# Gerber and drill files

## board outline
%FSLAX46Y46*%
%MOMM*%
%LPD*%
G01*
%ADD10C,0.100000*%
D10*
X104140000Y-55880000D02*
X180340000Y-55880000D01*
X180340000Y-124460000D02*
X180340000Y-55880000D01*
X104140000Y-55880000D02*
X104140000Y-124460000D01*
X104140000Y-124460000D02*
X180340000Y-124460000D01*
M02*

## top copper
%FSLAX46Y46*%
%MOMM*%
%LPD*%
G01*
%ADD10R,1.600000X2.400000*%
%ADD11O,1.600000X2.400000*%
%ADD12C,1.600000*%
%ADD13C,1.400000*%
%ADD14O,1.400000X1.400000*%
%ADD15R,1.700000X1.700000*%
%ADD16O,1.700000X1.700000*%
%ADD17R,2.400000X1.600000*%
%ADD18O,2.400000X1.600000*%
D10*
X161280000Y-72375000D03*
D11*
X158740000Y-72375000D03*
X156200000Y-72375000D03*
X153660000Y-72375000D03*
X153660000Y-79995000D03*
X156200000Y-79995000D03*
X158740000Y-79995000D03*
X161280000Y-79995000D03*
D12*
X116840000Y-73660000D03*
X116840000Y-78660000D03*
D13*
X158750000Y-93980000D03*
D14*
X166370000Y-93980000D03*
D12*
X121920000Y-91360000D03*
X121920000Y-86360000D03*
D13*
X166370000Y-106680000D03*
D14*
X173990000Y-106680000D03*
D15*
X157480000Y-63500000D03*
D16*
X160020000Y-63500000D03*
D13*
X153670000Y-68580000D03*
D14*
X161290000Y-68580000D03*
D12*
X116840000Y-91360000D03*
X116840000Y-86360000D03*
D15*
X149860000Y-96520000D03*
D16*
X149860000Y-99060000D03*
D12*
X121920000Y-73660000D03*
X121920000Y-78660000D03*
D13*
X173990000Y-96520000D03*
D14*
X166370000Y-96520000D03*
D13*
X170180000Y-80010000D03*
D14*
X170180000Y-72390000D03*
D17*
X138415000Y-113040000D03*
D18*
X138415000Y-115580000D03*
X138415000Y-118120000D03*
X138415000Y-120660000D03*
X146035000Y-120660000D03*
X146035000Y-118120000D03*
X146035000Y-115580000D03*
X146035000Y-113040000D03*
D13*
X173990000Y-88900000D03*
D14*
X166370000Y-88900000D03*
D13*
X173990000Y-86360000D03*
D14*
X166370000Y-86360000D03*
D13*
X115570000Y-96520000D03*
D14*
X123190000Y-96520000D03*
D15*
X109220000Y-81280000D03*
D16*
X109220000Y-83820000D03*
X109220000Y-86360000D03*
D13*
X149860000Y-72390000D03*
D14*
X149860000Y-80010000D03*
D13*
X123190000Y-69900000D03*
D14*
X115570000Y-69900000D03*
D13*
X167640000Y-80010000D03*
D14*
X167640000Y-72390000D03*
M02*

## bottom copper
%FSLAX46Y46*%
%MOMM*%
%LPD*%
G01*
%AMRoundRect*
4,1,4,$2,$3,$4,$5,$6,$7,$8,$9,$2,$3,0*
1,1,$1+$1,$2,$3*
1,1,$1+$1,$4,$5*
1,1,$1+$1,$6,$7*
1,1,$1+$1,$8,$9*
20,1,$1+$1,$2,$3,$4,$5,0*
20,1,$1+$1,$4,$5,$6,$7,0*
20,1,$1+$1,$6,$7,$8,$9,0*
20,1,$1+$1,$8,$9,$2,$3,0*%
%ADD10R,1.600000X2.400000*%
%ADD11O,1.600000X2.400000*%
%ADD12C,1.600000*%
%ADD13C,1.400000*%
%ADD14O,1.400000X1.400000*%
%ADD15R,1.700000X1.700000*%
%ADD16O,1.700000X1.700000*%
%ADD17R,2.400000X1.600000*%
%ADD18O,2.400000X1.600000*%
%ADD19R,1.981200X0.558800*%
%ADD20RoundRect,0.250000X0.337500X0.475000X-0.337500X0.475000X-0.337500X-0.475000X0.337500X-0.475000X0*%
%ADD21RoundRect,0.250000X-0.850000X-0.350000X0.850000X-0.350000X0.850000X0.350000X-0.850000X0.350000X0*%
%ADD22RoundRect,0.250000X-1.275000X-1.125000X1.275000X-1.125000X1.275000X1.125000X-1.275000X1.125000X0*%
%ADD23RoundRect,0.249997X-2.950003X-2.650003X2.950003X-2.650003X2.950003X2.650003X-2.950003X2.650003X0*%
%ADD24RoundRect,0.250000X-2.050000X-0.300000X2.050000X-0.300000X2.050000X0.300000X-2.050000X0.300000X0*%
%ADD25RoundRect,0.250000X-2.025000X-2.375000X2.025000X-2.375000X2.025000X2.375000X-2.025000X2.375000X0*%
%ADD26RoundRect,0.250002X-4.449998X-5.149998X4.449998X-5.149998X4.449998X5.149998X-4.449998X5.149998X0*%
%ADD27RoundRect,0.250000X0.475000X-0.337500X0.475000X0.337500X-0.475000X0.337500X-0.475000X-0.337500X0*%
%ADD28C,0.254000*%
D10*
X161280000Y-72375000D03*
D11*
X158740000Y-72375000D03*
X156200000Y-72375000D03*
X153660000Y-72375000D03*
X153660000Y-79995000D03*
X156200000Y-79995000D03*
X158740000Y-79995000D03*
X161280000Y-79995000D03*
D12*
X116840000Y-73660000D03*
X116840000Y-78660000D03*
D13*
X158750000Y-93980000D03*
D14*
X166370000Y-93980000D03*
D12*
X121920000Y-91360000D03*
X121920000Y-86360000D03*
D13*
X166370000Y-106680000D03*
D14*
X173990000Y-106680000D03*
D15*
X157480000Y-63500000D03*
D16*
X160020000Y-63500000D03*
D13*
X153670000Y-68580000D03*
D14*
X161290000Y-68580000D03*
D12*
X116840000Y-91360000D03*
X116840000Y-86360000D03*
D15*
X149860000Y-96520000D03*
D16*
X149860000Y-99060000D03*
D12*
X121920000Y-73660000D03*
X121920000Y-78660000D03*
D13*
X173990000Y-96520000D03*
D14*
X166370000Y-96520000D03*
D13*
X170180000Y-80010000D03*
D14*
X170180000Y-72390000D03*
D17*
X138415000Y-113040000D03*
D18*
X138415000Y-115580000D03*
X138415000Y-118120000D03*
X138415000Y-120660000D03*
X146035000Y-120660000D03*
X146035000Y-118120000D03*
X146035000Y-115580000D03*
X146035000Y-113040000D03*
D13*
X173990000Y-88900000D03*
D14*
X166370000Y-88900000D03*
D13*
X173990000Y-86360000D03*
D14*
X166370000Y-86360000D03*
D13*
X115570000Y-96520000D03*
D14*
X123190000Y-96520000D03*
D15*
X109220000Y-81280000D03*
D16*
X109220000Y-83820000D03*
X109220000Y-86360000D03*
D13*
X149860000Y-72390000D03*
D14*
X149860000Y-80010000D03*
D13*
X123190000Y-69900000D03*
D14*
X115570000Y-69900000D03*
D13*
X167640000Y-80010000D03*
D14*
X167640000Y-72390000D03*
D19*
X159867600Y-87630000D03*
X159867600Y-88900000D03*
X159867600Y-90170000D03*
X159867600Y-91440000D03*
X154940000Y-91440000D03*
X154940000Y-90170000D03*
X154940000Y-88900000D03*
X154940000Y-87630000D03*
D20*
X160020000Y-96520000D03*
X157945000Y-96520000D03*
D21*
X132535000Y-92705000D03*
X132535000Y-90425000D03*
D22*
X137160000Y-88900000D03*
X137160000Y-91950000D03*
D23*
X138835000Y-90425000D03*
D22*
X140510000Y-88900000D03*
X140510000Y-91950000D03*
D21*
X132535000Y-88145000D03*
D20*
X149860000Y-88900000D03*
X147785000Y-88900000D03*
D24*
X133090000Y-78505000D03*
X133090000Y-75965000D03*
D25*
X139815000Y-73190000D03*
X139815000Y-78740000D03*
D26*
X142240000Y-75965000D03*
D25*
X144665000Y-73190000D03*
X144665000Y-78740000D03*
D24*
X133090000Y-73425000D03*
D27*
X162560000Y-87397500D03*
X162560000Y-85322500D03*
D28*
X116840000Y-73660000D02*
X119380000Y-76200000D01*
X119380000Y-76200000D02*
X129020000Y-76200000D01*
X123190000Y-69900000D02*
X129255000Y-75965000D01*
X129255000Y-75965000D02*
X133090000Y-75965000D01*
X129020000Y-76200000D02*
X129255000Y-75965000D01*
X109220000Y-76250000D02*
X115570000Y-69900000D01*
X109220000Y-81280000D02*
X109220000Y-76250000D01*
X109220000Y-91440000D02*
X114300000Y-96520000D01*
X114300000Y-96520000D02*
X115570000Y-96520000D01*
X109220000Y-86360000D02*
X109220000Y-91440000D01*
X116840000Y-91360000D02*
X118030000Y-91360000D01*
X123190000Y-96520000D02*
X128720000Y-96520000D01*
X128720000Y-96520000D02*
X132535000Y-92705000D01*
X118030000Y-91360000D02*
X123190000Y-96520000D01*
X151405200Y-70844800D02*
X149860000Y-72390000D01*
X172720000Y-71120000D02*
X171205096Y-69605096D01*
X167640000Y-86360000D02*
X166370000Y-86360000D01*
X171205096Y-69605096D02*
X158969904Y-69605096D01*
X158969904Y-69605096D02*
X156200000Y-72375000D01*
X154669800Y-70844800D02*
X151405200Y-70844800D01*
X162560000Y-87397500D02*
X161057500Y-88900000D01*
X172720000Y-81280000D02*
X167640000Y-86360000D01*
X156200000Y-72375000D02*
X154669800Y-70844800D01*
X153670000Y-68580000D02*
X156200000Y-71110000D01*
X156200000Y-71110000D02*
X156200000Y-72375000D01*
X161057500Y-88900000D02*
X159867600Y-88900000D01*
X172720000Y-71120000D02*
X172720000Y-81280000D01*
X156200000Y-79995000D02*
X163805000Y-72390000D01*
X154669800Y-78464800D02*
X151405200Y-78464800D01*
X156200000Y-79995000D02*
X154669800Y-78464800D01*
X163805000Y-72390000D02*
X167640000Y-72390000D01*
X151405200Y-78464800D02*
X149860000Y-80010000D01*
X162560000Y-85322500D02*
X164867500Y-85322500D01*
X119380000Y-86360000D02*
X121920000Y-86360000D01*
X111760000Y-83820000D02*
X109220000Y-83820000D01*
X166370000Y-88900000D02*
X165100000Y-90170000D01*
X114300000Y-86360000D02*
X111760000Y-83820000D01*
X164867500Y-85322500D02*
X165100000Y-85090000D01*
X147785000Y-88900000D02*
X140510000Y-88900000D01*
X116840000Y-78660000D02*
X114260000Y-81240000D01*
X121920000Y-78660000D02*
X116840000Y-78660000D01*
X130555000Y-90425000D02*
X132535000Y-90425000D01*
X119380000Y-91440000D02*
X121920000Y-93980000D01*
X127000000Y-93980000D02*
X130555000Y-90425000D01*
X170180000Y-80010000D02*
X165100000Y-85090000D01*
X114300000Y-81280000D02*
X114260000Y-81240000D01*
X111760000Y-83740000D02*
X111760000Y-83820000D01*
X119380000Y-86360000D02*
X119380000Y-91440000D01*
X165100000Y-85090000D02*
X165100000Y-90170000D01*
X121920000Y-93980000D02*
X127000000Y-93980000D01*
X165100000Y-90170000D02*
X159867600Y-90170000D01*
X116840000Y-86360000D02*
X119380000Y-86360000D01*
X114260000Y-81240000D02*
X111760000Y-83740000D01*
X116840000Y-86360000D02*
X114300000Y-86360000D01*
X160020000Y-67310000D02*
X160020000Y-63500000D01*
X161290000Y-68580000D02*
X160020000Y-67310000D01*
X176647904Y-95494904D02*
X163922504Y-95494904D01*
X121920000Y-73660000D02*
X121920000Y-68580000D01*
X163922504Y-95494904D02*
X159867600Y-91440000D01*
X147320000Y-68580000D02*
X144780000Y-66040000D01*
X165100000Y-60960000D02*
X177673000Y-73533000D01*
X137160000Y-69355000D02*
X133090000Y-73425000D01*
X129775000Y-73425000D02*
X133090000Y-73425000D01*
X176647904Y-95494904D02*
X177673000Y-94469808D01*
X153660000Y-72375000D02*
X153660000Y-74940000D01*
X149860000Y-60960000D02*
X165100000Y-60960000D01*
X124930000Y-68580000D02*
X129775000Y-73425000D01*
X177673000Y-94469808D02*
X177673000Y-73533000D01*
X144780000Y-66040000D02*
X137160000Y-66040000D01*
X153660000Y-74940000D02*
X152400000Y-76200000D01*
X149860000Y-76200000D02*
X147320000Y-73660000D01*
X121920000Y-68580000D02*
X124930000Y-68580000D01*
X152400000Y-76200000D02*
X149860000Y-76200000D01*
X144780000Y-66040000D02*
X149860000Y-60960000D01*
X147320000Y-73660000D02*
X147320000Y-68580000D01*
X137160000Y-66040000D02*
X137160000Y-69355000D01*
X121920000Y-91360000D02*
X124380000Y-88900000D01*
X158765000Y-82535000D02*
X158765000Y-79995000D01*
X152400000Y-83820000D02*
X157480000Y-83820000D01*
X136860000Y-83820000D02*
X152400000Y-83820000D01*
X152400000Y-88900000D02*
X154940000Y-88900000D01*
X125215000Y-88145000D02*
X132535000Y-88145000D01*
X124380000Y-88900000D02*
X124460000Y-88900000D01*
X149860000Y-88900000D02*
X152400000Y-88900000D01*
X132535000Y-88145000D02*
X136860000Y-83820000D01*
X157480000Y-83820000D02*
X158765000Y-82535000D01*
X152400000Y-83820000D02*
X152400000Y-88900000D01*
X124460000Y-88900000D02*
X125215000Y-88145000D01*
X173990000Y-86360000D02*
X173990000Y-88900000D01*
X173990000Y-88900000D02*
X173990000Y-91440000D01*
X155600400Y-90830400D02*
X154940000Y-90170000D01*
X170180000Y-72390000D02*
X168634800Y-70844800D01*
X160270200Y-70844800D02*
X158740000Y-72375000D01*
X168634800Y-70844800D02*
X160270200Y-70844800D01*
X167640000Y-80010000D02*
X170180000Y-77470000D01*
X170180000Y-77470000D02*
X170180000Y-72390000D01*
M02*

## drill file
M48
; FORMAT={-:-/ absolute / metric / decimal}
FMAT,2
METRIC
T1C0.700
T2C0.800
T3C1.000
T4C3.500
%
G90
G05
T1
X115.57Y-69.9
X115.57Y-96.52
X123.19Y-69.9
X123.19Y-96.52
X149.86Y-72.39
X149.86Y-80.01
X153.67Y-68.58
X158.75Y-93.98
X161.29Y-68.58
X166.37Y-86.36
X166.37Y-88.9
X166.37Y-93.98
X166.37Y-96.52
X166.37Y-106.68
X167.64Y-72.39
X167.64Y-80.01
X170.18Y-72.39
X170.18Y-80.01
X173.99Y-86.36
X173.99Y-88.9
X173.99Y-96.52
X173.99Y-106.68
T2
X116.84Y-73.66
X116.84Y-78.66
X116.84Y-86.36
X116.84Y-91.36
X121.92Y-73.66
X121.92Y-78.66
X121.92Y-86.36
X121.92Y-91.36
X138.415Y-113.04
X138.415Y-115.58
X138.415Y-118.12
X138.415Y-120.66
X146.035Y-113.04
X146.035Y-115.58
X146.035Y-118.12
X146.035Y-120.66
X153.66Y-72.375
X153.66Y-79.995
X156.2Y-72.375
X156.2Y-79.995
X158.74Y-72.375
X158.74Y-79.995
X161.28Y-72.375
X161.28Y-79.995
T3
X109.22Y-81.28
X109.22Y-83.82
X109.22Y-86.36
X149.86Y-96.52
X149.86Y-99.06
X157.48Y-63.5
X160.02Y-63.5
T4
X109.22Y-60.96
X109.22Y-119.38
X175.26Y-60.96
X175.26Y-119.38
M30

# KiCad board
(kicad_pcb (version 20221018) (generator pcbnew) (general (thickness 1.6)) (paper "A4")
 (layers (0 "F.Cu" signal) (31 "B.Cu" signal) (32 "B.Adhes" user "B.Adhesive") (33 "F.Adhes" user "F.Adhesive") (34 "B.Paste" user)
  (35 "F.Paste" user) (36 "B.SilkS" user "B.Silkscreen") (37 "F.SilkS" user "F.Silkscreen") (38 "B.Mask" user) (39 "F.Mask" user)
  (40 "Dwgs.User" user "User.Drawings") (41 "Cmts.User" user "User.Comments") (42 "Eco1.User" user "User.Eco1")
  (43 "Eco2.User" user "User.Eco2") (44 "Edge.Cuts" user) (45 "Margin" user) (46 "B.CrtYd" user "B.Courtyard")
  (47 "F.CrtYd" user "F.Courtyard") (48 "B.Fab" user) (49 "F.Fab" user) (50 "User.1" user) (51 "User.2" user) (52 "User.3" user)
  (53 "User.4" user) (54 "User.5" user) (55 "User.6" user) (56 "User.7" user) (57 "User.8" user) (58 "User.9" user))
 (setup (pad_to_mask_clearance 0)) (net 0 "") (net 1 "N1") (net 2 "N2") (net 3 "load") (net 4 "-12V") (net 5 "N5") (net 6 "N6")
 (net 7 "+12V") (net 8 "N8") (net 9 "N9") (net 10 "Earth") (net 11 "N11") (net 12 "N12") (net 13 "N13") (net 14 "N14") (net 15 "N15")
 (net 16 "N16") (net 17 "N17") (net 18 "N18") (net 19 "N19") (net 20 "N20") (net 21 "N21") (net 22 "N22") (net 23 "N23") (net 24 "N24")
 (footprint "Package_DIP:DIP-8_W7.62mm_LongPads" (layer "F.Cu") (at 161.28 72.375 -90)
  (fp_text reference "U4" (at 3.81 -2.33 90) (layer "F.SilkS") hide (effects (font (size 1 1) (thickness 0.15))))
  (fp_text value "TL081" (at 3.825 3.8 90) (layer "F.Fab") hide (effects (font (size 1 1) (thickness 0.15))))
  (pad "1" thru_hole rect (at 0 0 270) (size 2.4 1.6) (drill 0.8) (layers "*.Cu" "*.Mask") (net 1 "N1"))
  (pad "2" thru_hole oval (at 0 2.54 270) (size 2.4 1.6) (drill 0.8) (layers "*.Cu" "*.Mask") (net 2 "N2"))
  (pad "3" thru_hole oval (at 0 5.08 270) (size 2.4 1.6) (drill 0.8) (layers "*.Cu" "*.Mask") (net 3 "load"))
  (pad "4" thru_hole oval (at 0 7.62 270) (size 2.4 1.6) (drill 0.8) (layers "*.Cu" "*.Mask") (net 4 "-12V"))
  (pad "5" thru_hole oval (at 7.62 7.62 270) (size 2.4 1.6) (drill 0.8) (layers "*.Cu" "*.Mask") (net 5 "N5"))
  (pad "6" thru_hole oval (at 7.62 5.08 270) (size 2.4 1.6) (drill 0.8) (layers "*.Cu" "*.Mask") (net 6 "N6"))
  (pad "7" thru_hole oval (at 7.62 2.54 270) (size 2.4 1.6) (drill 0.8) (layers "*.Cu" "*.Mask") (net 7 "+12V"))
  (pad "8" thru_hole oval (at 7.62 0 270) (size 2.4 1.6) (drill 0.8) (layers "*.Cu" "*.Mask") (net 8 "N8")))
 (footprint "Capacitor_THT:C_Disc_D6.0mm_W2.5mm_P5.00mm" (layer "F.Cu") (at 116.84 73.66 -90)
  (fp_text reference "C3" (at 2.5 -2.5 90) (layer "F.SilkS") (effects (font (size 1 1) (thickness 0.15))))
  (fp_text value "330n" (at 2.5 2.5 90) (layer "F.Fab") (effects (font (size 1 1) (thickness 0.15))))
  (pad "1" thru_hole circle (at 0 0 270) (size 1.6 1.6) (drill 0.8) (layers "*.Cu" "*.Mask") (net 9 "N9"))
  (pad "2" thru_hole circle (at 5 0 270) (size 1.6 1.6) (drill 0.8) (layers "*.Cu" "*.Mask") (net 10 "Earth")))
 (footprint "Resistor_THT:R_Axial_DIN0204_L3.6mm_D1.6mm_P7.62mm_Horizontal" (layer "F.Cu") (at 158.75 93.98)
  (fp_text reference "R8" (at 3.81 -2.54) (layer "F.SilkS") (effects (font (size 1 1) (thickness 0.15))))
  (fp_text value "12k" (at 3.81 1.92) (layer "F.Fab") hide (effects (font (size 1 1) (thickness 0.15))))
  (pad "1" thru_hole circle (at 0 0) (size 1.4 1.4) (drill 0.7) (layers "*.Cu" "*.Mask") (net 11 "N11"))
  (pad "2" thru_hole oval (at 7.62 0) (size 1.4 1.4) (drill 0.7) (layers "*.Cu" "*.Mask") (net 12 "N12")))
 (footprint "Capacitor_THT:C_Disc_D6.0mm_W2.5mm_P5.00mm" (layer "F.Cu") (at 121.92 91.36 90)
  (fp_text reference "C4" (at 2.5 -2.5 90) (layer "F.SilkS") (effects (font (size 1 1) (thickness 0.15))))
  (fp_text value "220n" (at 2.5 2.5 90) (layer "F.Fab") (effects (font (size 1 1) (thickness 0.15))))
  (pad "1" thru_hole circle (at 0 0 90) (size 1.6 1.6) (drill 0.8) (layers "*.Cu" "*.Mask") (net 7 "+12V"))
  (pad "2" thru_hole circle (at 5 0 90) (size 1.6 1.6) (drill 0.8) (layers "*.Cu" "*.Mask") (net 10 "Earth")))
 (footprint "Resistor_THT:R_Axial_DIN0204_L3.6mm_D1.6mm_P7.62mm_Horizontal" (layer "F.Cu") (at 166.37 106.68)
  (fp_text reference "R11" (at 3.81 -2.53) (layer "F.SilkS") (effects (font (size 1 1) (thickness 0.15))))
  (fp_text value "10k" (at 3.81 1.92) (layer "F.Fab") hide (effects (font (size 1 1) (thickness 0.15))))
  (pad "1" thru_hole circle (at 0 0) (size 1.4 1.4) (drill 0.7) (layers "*.Cu" "*.Mask") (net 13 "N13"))
  (pad "2" thru_hole oval (at 7.62 0) (size 1.4 1.4) (drill 0.7) (layers "*.Cu" "*.Mask") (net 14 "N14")))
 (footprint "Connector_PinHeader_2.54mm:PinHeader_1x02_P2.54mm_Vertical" (layer "F.Cu") (at 157.48 63.5 90)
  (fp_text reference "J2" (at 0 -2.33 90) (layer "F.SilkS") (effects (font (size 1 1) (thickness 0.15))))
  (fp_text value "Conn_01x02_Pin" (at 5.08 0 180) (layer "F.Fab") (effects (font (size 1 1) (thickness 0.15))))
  (pad "1" thru_hole rect (at 0 0 90) (size 1.7 1.7) (drill 1) (layers "*.Cu" "*.Mask") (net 10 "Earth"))
  (pad "2" thru_hole oval (at 0 2.54 90) (size 1.7 1.7) (drill 1) (layers "*.Cu" "*.Mask") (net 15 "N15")))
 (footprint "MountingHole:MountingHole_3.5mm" (layer "F.Cu") (at 175.26 60.96)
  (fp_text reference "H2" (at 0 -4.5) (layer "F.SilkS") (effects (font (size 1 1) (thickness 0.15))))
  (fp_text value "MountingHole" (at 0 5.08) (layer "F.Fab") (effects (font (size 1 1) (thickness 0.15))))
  (pad "" np_thru_hole circle (at 0 0) (size 3.5 3.5) (drill 3.5) (layers "*.Cu" "*.Mask")))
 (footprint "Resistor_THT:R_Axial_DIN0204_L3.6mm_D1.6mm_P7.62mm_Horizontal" (layer "F.Cu") (at 153.67 68.58)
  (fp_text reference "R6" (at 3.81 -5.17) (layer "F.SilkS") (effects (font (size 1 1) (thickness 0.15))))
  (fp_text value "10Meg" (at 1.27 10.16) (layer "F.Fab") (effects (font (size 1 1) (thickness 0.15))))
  (pad "1" thru_hole circle (at 0 0) (size 1.4 1.4) (drill 0.7) (layers "*.Cu" "*.Mask") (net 3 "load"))
  (pad "2" thru_hole oval (at 7.62 0) (size 1.4 1.4) (drill 0.7) (layers "*.Cu" "*.Mask") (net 15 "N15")))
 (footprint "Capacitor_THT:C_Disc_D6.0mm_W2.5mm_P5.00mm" (layer "F.Cu") (at 116.84 91.36 90)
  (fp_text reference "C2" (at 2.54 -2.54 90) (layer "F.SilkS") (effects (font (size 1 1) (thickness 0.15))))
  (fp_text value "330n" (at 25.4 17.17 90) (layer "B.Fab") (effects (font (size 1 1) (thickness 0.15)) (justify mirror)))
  (pad "1" thru_hole circle (at 0 0 90) (size 1.6 1.6) (drill 0.8) (layers "*.Cu" "*.Mask") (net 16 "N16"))
  (pad "2" thru_hole circle (at 5 0 90) (size 1.6 1.6) (drill 0.8) (layers "*.Cu" "*.Mask") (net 10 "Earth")))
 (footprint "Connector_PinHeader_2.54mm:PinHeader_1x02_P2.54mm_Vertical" (layer "F.Cu") (at 149.86 96.52)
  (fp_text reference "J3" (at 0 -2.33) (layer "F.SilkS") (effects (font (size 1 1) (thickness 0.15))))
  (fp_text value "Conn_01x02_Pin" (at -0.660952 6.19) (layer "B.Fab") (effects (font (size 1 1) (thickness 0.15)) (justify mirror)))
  (pad "1" thru_hole rect (at 0 0) (size 1.7 1.7) (drill 1) (layers "*.Cu" "*.Mask") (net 13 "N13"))
  (pad "2" thru_hole oval (at 0 2.54) (size 1.7 1.7) (drill 1) (layers "*.Cu" "*.Mask") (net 10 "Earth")))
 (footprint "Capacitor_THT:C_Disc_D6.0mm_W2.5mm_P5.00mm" (layer "F.Cu") (at 121.92 73.66 -90)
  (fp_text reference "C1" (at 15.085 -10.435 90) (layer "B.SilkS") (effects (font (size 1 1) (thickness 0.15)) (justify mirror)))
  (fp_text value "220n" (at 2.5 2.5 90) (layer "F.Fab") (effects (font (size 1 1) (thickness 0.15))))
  (pad "1" thru_hole circle (at 0 0 270) (size 1.6 1.6) (drill 0.8) (layers "*.Cu" "*.Mask") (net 4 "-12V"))
  (pad "2" thru_hole circle (at 5 0 270) (size 1.6 1.6) (drill 0.8) (layers "*.Cu" "*.Mask") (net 10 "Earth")))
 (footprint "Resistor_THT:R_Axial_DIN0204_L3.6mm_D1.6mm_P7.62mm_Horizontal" (layer "F.Cu") (at 173.99 96.52 180)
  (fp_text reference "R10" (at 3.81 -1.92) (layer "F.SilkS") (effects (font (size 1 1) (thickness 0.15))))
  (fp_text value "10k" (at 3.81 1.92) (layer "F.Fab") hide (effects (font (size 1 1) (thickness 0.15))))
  (pad "1" thru_hole circle (at 0 0 180) (size 1.4 1.4) (drill 0.7) (layers "*.Cu" "*.Mask") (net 14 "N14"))
  (pad "2" thru_hole oval (at 7.62 0 180) (size 1.4 1.4) (drill 0.7) (layers "*.Cu" "*.Mask") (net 11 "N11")))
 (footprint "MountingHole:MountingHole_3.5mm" (layer "F.Cu") (at 109.22 119.38)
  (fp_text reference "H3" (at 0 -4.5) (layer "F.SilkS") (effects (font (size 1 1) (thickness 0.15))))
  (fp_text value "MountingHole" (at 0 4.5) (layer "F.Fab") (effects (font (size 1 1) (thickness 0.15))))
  (pad "" np_thru_hole circle (at 0 0) (size 3.5 3.5) (drill 3.5) (layers "*.Cu" "*.Mask")))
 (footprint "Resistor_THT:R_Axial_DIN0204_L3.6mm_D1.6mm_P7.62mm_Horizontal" (layer "F.Cu") (at 170.18 80.01 90)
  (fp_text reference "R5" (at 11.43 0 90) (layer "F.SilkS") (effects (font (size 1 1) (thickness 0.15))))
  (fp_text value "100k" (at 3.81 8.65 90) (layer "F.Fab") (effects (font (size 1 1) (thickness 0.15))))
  (pad "1" thru_hole circle (at 0 0 90) (size 1.4 1.4) (drill 0.7) (layers "*.Cu" "*.Mask") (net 10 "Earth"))
  (pad "2" thru_hole oval (at 7.62 0 90) (size 1.4 1.4) (drill 0.7) (layers "*.Cu" "*.Mask") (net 2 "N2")))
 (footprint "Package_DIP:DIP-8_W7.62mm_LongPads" (layer "F.Cu") (at 138.415 113.04)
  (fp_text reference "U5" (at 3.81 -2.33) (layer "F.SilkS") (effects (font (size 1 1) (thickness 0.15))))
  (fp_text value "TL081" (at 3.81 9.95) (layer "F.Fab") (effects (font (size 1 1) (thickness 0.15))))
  (pad "1" thru_hole rect (at 0 0) (size 2.4 1.6) (drill 0.8) (layers "*.Cu" "*.Mask") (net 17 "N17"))
  (pad "2" thru_hole oval (at 0 2.54) (size 2.4 1.6) (drill 0.8) (layers "*.Cu" "*.Mask") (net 10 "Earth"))
  (pad "3" thru_hole oval (at 0 5.08) (size 2.4 1.6) (drill 0.8) (layers "*.Cu" "*.Mask") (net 14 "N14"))
  (pad "4" thru_hole oval (at 0 7.62) (size 2.4 1.6) (drill 0.8) (layers "*.Cu" "*.Mask") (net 4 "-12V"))
  (pad "5" thru_hole oval (at 7.62 7.62) (size 2.4 1.6) (drill 0.8) (layers "*.Cu" "*.Mask") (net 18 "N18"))
  (pad "6" thru_hole oval (at 7.62 5.08) (size 2.4 1.6) (drill 0.8) (layers "*.Cu" "*.Mask") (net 13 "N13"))
  (pad "7" thru_hole oval (at 7.62 2.54) (size 2.4 1.6) (drill 0.8) (layers "*.Cu" "*.Mask") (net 7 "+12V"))
  (pad "8" thru_hole oval (at 7.62 0) (size 2.4 1.6) (drill 0.8) (layers "*.Cu" "*.Mask") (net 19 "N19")))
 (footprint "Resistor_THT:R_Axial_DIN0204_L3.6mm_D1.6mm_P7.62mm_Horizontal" (layer "F.Cu") (at 173.99 88.9 180)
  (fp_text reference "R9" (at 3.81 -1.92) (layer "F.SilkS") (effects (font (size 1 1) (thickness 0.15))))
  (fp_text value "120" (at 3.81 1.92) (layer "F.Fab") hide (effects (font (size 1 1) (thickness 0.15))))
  (pad "1" thru_hole circle (at 0 0 180) (size 1.4 1.4) (drill 0.7) (layers "*.Cu" "*.Mask") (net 12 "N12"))
  (pad "2" thru_hole oval (at 7.62 0 180) (size 1.4 1.4) (drill 0.7) (layers "*.Cu" "*.Mask") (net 10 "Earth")))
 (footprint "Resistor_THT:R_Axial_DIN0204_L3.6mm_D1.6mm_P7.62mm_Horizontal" (layer "F.Cu") (at 173.99 86.36 180)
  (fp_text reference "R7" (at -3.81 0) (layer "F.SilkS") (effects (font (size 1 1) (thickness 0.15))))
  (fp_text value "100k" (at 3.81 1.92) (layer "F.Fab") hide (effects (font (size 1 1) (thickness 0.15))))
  (pad "1" thru_hole circle (at 0 0 180) (size 1.4 1.4) (drill 0.7) (layers "*.Cu" "*.Mask") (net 12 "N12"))
  (pad "2" thru_hole oval (at 7.62 0 180) (size 1.4 1.4) (drill 0.7) (layers "*.Cu" "*.Mask") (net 3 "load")))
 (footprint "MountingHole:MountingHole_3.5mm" (layer "F.Cu") (at 109.22 60.96)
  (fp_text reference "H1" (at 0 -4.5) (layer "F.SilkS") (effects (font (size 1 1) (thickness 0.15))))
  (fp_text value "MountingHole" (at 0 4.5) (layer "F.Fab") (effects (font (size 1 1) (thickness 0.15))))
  (pad "" np_thru_hole circle (at 0 0) (size 3.5 3.5) (drill 3.5) (layers "*.Cu" "*.Mask")))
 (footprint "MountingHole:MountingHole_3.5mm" (layer "F.Cu") (at 175.26 119.38)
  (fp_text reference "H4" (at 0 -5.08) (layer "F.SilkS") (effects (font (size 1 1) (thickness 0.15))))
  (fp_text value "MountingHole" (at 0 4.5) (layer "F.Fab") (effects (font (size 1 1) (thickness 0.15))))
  (pad "" np_thru_hole circle (at 0 0) (size 3.5 3.5) (drill 3.5) (layers "*.Cu" "*.Mask")))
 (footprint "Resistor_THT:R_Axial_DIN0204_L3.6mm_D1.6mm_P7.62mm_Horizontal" (layer "F.Cu") (at 115.57 96.52)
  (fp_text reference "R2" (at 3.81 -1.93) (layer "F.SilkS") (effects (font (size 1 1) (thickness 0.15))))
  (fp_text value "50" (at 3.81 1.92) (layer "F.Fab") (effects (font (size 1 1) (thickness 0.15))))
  (pad "1" thru_hole circle (at 0 0) (size 1.4 1.4) (drill 0.7) (layers "*.Cu" "*.Mask") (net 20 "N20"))
  (pad "2" thru_hole oval (at 7.62 0) (size 1.4 1.4) (drill 0.7) (layers "*.Cu" "*.Mask") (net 16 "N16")))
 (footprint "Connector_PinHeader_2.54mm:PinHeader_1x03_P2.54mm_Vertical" (layer "F.Cu") (at 109.22 81.28)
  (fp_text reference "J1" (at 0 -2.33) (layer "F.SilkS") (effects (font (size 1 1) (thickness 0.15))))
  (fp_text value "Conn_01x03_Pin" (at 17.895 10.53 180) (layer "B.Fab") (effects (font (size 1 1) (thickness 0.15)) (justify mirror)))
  (pad "1" thru_hole rect (at 0 0) (size 1.7 1.7) (drill 1) (layers "*.Cu" "*.Mask") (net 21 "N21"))
  (pad "2" thru_hole oval (at 0 2.54) (size 1.7 1.7) (drill 1) (layers "*.Cu" "*.Mask") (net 10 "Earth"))
  (pad "3" thru_hole oval (at 0 5.08) (size 1.7 1.7) (drill 1) (layers "*.Cu" "*.Mask") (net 20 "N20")))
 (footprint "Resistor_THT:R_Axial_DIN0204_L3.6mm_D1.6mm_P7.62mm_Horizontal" (layer "F.Cu") (at 149.86 72.39 -90)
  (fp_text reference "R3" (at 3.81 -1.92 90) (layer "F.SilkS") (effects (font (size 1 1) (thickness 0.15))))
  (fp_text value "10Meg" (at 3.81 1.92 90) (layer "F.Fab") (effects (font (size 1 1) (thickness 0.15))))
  (pad "1" thru_hole circle (at 0 0 270) (size 1.4 1.4) (drill 0.7) (layers "*.Cu" "*.Mask") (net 3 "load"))
  (pad "2" thru_hole oval (at 7.62 0 270) (size 1.4 1.4) (drill 0.7) (layers "*.Cu" "*.Mask") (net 6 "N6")))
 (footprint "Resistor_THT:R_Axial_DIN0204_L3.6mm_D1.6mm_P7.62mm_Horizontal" (layer "F.Cu") (at 123.19 69.9 180)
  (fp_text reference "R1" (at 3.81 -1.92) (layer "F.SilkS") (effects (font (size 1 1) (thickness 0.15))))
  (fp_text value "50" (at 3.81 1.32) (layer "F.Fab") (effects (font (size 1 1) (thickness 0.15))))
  (pad "1" thru_hole circle (at 0 0 180) (size 1.4 1.4) (drill 0.7) (layers "*.Cu" "*.Mask") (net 9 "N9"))
  (pad "2" thru_hole oval (at 7.62 0 180) (size 1.4 1.4) (drill 0.7) (layers "*.Cu" "*.Mask") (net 21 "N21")))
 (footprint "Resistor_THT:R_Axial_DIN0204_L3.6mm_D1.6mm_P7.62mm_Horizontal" (layer "F.Cu") (at 167.64 80.01 90)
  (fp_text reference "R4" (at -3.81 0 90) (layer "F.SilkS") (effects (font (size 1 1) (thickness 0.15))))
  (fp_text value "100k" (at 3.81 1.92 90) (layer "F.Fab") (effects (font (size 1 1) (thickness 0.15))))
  (pad "1" thru_hole circle (at 0 0 90) (size 1.4 1.4) (drill 0.7) (layers "*.Cu" "*.Mask") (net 2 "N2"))
  (pad "2" thru_hole oval (at 7.62 0 90) (size 1.4 1.4) (drill 0.7) (layers "*.Cu" "*.Mask") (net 6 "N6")))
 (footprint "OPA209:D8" (layer "B.Cu") (at 157.4038 89.535 180)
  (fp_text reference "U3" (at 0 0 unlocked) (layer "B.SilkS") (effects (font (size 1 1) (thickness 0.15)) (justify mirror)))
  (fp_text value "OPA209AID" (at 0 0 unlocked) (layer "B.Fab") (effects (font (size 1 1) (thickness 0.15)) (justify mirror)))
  (pad "1" smd rect (at -2.4638 1.905 180) (size 1.9812 0.5588) (layers "B.Cu" "B.Paste" "B.Mask") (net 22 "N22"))
  (pad "2" smd rect (at -2.4638 0.635 180) (size 1.9812 0.5588) (layers "B.Cu" "B.Paste" "B.Mask") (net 3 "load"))
  (pad "3" smd rect (at -2.4638 -0.635 180) (size 1.9812 0.5588) (layers "B.Cu" "B.Paste" "B.Mask") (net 10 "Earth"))
  (pad "4" smd rect (at -2.4638 -1.905 180) (size 1.9812 0.5588) (layers "B.Cu" "B.Paste" "B.Mask") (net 4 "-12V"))
  (pad "5" smd rect (at 2.4638 -1.905 180) (size 1.9812 0.5588) (layers "B.Cu" "B.Paste" "B.Mask") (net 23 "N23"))
  (pad "6" smd rect (at 2.4638 -0.635 180) (size 1.9812 0.5588) (layers "B.Cu" "B.Paste" "B.Mask") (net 11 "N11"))
  (pad "7" smd rect (at 2.4638 0.635 180) (size 1.9812 0.5588) (layers "B.Cu" "B.Paste" "B.Mask") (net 7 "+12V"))
  (pad "8" smd rect (at 2.4638 1.905 180) (size 1.9812 0.5588) (layers "B.Cu" "B.Paste" "B.Mask") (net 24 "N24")))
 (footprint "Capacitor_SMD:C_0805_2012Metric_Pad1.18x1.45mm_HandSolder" (layer "B.Cu") (at 158.9825 96.52 180)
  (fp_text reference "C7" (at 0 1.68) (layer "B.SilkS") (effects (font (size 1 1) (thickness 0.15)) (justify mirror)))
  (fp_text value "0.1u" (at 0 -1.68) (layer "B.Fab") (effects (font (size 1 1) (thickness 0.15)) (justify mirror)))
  (pad "1" smd roundrect (at -1.0375 0 180) (size 1.175 1.45) (layers "B.Cu" "B.Paste" "B.Mask") (roundrect_rratio 0.2127659574)
   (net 4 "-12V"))
  (pad "2" smd roundrect (at 1.0375 0 180) (size 1.175 1.45) (layers "B.Cu" "B.Paste" "B.Mask") (roundrect_rratio 0.2127659574)
   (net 10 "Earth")))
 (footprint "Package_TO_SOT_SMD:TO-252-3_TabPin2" (layer "B.Cu") (at 137.575 90.425)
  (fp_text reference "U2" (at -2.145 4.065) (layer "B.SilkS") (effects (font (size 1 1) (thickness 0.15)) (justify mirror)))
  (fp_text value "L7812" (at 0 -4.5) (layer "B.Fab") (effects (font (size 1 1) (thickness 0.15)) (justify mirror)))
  (pad "1" smd roundrect (at -5.04 2.28) (size 2.2 1.2) (layers "B.Cu" "B.Paste" "B.Mask") (roundrect_rratio 0.2083333333) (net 16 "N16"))
  (pad "2" smd roundrect (at -5.04 0) (size 2.2 1.2) (layers "B.Cu" "B.Paste" "B.Mask") (roundrect_rratio 0.2083333333) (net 10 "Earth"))
  (pad "2" smd roundrect (at -0.415 -1.525) (size 3.05 2.75) (layers "B.Cu" "B.Paste") (roundrect_rratio 0.09090909091) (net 10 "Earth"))
  (pad "2" smd roundrect (at -0.415 1.525) (size 3.05 2.75) (layers "B.Cu" "B.Paste") (roundrect_rratio 0.09090909091) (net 10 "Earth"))
  (pad "2" smd roundrect (at 1.26 0) (size 6.4 5.8) (layers "B.Cu" "B.Mask") (roundrect_rratio 0.04310293103) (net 10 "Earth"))
  (pad "2" smd roundrect (at 2.935 -1.525) (size 3.05 2.75) (layers "B.Cu" "B.Paste") (roundrect_rratio 0.09090909091) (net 10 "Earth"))
  (pad "2" smd roundrect (at 2.935 1.525) (size 3.05 2.75) (layers "B.Cu" "B.Paste") (roundrect_rratio 0.09090909091) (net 10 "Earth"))
  (pad "3" smd roundrect (at -5.04 -2.28) (size 2.2 1.2) (layers "B.Cu" "B.Paste" "B.Mask") (roundrect_rratio 0.2083333333) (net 7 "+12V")))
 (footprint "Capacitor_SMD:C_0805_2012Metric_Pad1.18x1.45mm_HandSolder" (layer "B.Cu") (at 148.8225 88.9 180)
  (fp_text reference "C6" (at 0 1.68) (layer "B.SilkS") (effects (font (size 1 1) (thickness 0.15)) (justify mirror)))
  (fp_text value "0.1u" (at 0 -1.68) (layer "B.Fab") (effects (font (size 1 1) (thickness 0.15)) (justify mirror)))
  (pad "1" smd roundrect (at -1.0375 0 180) (size 1.175 1.45) (layers "B.Cu" "B.Paste" "B.Mask") (roundrect_rratio 0.2127659574)
   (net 7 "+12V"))
  (pad "2" smd roundrect (at 1.0375 0 180) (size 1.175 1.45) (layers "B.Cu" "B.Paste" "B.Mask") (roundrect_rratio 0.2127659574)
   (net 10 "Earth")))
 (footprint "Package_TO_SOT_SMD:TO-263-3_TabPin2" (layer "B.Cu") (at 140.74 75.965)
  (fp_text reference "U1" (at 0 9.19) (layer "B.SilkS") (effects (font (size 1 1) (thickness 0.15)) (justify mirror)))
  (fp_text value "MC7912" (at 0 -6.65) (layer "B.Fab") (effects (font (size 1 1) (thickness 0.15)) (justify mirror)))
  (pad "1" smd roundrect (at -7.65 2.54) (size 4.6 1.1) (layers "B.Cu" "B.Paste" "B.Mask") (roundrect_rratio 0.2272727273) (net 10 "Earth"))
  (pad "2" smd roundrect (at -7.65 0) (size 4.6 1.1) (layers "B.Cu" "B.Paste" "B.Mask") (roundrect_rratio 0.2272727273) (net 9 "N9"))
  (pad "2" smd roundrect (at -0.925 -2.775) (size 4.55 5.25) (layers "B.Cu" "B.Paste") (roundrect_rratio 0.05494505495) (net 9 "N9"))
  (pad "2" smd roundrect (at -0.925 2.775) (size 4.55 5.25) (layers "B.Cu" "B.Paste") (roundrect_rratio 0.05494505495) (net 9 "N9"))
  (pad "2" smd roundrect (at 1.5 0) (size 9.4 10.8) (layers "B.Cu" "B.Mask") (roundrect_rratio 0.02659595745) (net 9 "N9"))
  (pad "2" smd roundrect (at 3.925 -2.775) (size 4.55 5.25) (layers "B.Cu" "B.Paste") (roundrect_rratio 0.05494505495) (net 9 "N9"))
  (pad "2" smd roundrect (at 3.925 2.775) (size 4.55 5.25) (layers "B.Cu" "B.Paste") (roundrect_rratio 0.05494505495) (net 9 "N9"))
  (pad "3" smd roundrect (at -7.65 -2.54) (size 4.6 1.1) (layers "B.Cu" "B.Paste" "B.Mask") (roundrect_rratio 0.2272727273) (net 4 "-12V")))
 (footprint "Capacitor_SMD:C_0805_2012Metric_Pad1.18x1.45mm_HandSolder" (layer "B.Cu") (at 162.56 86.36 90)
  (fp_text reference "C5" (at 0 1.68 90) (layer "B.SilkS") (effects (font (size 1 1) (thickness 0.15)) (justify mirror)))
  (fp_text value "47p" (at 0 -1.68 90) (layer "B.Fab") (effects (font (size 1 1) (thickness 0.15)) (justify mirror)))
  (pad "1" smd roundrect (at -1.0375 0 90) (size 1.175 1.45) (layers "B.Cu" "B.Paste" "B.Mask") (roundrect_rratio 0.2127659574)
   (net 3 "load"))
  (pad "2" smd roundrect (at 1.0375 0 90) (size 1.175 1.45) (layers "B.Cu" "B.Paste" "B.Mask") (roundrect_rratio 0.2127659574)
   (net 10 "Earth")))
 (gr_line (start 104.14 55.88) (end 180.34 55.88) (stroke (width 0.1) (type default)) (layer "Edge.Cuts"))
 (gr_line (start 180.34 124.46) (end 180.34 55.88) (stroke (width 0.1) (type default)) (layer "Edge.Cuts"))
 (gr_line (start 104.14 55.88) (end 104.14 124.46) (stroke (width 0.1) (type default)) (layer "Edge.Cuts"))
 (gr_line (start 104.14 124.46) (end 180.34 124.46) (stroke (width 0.1) (type default)) (layer "Edge.Cuts"))
 (segment (start 116.84 73.66) (end 119.38 76.2) (width 0.254) (layer "B.Cu") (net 9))
 (segment (start 119.38 76.2) (end 129.02 76.2) (width 0.254) (layer "B.Cu") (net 9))
 (segment (start 123.19 69.9) (end 129.255 75.965) (width 0.254) (layer "B.Cu") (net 9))
 (segment (start 129.255 75.965) (end 133.09 75.965) (width 0.254) (layer "B.Cu") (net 9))
 (segment (start 129.02 76.2) (end 129.255 75.965) (width 0.254) (layer "B.Cu") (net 9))
 (segment (start 109.22 76.25) (end 115.57 69.9) (width 0.254) (layer "B.Cu") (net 21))
 (segment (start 109.22 81.28) (end 109.22 76.25) (width 0.254) (layer "B.Cu") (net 21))
 (segment (start 109.22 91.44) (end 114.3 96.52) (width 0.254) (layer "B.Cu") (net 20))
 (segment (start 114.3 96.52) (end 115.57 96.52) (width 0.254) (layer "B.Cu") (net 20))
 (segment (start 109.22 86.36) (end 109.22 91.44) (width 0.254) (layer "B.Cu") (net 20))
 (segment (start 116.84 91.36) (end 118.03 91.36) (width 0.254) (layer "B.Cu") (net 16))
 (segment (start 123.19 96.52) (end 128.72 96.52) (width 0.254) (layer "B.Cu") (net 16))
 (segment (start 128.72 96.52) (end 132.535 92.705) (width 0.254) (layer "B.Cu") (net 16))
 (segment (start 118.03 91.36) (end 123.19 96.52) (width 0.254) (layer "B.Cu") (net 16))
 (segment (start 151.4052 70.8448) (end 149.86 72.39) (width 0.254) (layer "B.Cu") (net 3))
 (segment (start 172.72 71.12) (end 171.205096 69.605096) (width 0.254) (layer "B.Cu") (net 3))
 (segment (start 167.64 86.36) (end 166.37 86.36) (width 0.254) (layer "B.Cu") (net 3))
 (segment (start 171.205096 69.605096) (end 158.969904 69.605096) (width 0.254) (layer "B.Cu") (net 3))
 (segment (start 158.969904 69.605096) (end 156.2 72.375) (width 0.254) (layer "B.Cu") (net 3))
 (segment (start 154.6698 70.8448) (end 151.4052 70.8448) (width 0.254) (layer "B.Cu") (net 3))
 (segment (start 162.56 87.3975) (end 161.0575 88.9) (width 0.254) (layer "B.Cu") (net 3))
 (segment (start 172.72 81.28) (end 167.64 86.36) (width 0.254) (layer "B.Cu") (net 3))
 (segment (start 156.2 72.375) (end 154.6698 70.8448) (width 0.254) (layer "B.Cu") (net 3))
 (segment (start 153.67 68.58) (end 156.2 71.11) (width 0.254) (layer "B.Cu") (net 3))
 (segment (start 156.2 71.11) (end 156.2 72.375) (width 0.254) (layer "B.Cu") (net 3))
 (segment (start 161.0575 88.9) (end 159.8676 88.9) (width 0.254) (layer "B.Cu") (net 3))
 (segment (start 172.72 71.12) (end 172.72 81.28) (width 0.254) (layer "B.Cu") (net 3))
 (segment (start 156.2 79.995) (end 163.805 72.39) (width 0.254) (layer "B.Cu") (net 6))
 (segment (start 154.6698 78.4648) (end 151.4052 78.4648) (width 0.254) (layer "B.Cu") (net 6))
 (segment (start 156.2 79.995) (end 154.6698 78.4648) (width 0.254) (layer "B.Cu") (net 6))
 (segment (start 163.805 72.39) (end 167.64 72.39) (width 0.254) (layer "B.Cu") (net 6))
 (segment (start 151.4052 78.4648) (end 149.86 80.01) (width 0.254) (layer "B.Cu") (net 6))
 (segment (start 162.56 85.3225) (end 164.8675 85.3225) (width 0.254) (layer "B.Cu") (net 10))
 (segment (start 119.38 86.36) (end 121.92 86.36) (width 0.254) (layer "B.Cu") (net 10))
 (segment (start 111.76 83.82) (end 109.22 83.82) (width 0.254) (layer "B.Cu") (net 10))
 (segment (start 166.37 88.9) (end 165.1 90.17) (width 0.254) (layer "B.Cu") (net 10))
 (segment (start 114.3 86.36) (end 111.76 83.82) (width 0.254) (layer "B.Cu") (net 10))
 (segment (start 164.8675 85.3225) (end 165.1 85.09) (width 0.254) (layer "B.Cu") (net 10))
 (segment (start 147.785 88.9) (end 140.51 88.9) (width 0.254) (layer "B.Cu") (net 10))
 (segment (start 116.84 78.66) (end 114.26 81.24) (width 0.254) (layer "B.Cu") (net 10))
 (segment (start 121.92 78.66) (end 116.84 78.66) (width 0.254) (layer "B.Cu") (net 10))
 (segment (start 130.555 90.425) (end 132.535 90.425) (width 0.254) (layer "B.Cu") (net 10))
 (segment (start 119.38 91.44) (end 121.92 93.98) (width 0.254) (layer "B.Cu") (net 10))
 (segment (start 127 93.98) (end 130.555 90.425) (width 0.254) (layer "B.Cu") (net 10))
 (segment (start 170.18 80.01) (end 165.1 85.09) (width 0.254) (layer "B.Cu") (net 10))
 (segment (start 114.3 81.28) (end 114.26 81.24) (width 0.254) (layer "B.Cu") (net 10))
 (segment (start 111.76 83.74) (end 111.76 83.82) (width 0.254) (layer "B.Cu") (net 10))
 (segment (start 119.38 86.36) (end 119.38 91.44) (width 0.254) (layer "B.Cu") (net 10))
 (segment (start 165.1 85.09) (end 165.1 90.17) (width 0.254) (layer "B.Cu") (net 10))
 (segment (start 121.92 93.98) (end 127 93.98) (width 0.254) (layer "B.Cu") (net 10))
 (segment (start 165.1 90.17) (end 159.8676 90.17) (width 0.254) (layer "B.Cu") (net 10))
 (segment (start 116.84 86.36) (end 119.38 86.36) (width 0.254) (layer "B.Cu") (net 10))
 (segment (start 114.26 81.24) (end 111.76 83.74) (width 0.254) (layer "B.Cu") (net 10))
 (segment (start 116.84 86.36) (end 114.3 86.36) (width 0.254) (layer "B.Cu") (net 10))
 (segment (start 160.02 67.31) (end 160.02 63.5) (width 0.254) (layer "B.Cu") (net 15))
 (segment (start 161.29 68.58) (end 160.02 67.31) (width 0.254) (layer "B.Cu") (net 15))
 (segment (start 176.647904 95.494904) (end 163.922504 95.494904) (width 0.254) (layer "B.Cu") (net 4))
 (segment (start 121.92 73.66) (end 121.92 68.58) (width 0.254) (layer "B.Cu") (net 4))
 (segment (start 163.922504 95.494904) (end 159.8676 91.44) (width 0.254) (layer "B.Cu") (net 4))
 (segment (start 147.32 68.58) (end 144.78 66.04) (width 0.254) (layer "B.Cu") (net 4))
 (segment (start 165.1 60.96) (end 177.673 73.533) (width 0.254) (layer "B.Cu") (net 4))
 (segment (start 137.16 69.355) (end 133.09 73.425) (width 0.254) (layer "B.Cu") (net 4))
 (segment (start 129.775 73.425) (end 133.09 73.425) (width 0.254) (layer "B.Cu") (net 4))
 (segment (start 176.647904 95.494904) (end 177.673 94.469808) (width 0.254) (layer "B.Cu") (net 4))
 (segment (start 153.66 72.375) (end 153.66 74.94) (width 0.254) (layer "B.Cu") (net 4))
 (segment (start 149.86 60.96) (end 165.1 60.96) (width 0.254) (layer "B.Cu") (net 4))
 (segment (start 124.93 68.58) (end 129.775 73.425) (width 0.254) (layer "B.Cu") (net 4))
 (segment (start 177.673 94.469808) (end 177.673 73.533) (width 0.254) (layer "B.Cu") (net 4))
 (segment (start 144.78 66.04) (end 137.16 66.04) (width 0.254) (layer "B.Cu") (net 4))
 (segment (start 153.66 74.94) (end 152.4 76.2) (width 0.254) (layer "B.Cu") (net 4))
 (segment (start 149.86 76.2) (end 147.32 73.66) (width 0.254) (layer "B.Cu") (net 4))
 (segment (start 121.92 68.58) (end 124.93 68.58) (width 0.254) (layer "B.Cu") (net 4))
 (segment (start 152.4 76.2) (end 149.86 76.2) (width 0.254) (layer "B.Cu") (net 4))
 (segment (start 144.78 66.04) (end 149.86 60.96) (width 0.254) (layer "B.Cu") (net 4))
 (segment (start 147.32 73.66) (end 147.32 68.58) (width 0.254) (layer "B.Cu") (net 4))
 (segment (start 137.16 66.04) (end 137.16 69.355) (width 0.254) (layer "B.Cu") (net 4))
 (segment (start 121.92 91.36) (end 124.38 88.9) (width 0.254) (layer "B.Cu") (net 7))
 (segment (start 158.765 82.535) (end 158.765 79.995) (width 0.254) (layer "B.Cu") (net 7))
 (segment (start 152.4 83.82) (end 157.48 83.82) (width 0.254) (layer "B.Cu") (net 7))
 (segment (start 136.86 83.82) (end 152.4 83.82) (width 0.254) (layer "B.Cu") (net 7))
 (segment (start 152.4 88.9) (end 154.94 88.9) (width 0.254) (layer "B.Cu") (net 7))
 (segment (start 125.215 88.145) (end 132.535 88.145) (width 0.254) (layer "B.Cu") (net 7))
 (segment (start 124.38 88.9) (end 124.46 88.9) (width 0.254) (layer "B.Cu") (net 7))
 (segment (start 149.86 88.9) (end 152.4 88.9) (width 0.254) (layer "B.Cu") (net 7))
 (segment (start 132.535 88.145) (end 136.86 83.82) (width 0.254) (layer "B.Cu") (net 7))
 (segment (start 157.48 83.82) (end 158.765 82.535) (width 0.254) (layer "B.Cu") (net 7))
 (segment (start 152.4 83.82) (end 152.4 88.9) (width 0.254) (layer "B.Cu") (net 7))
 (segment (start 124.46 88.9) (end 125.215 88.145) (width 0.254) (layer "B.Cu") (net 7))
 (segment (start 173.99 86.36) (end 173.99 88.9) (width 0.254) (layer "B.Cu") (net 12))
 (segment (start 173.99 88.9) (end 173.99 91.44) (width 0.254) (layer "B.Cu") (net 12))
 (segment (start 155.6004 90.8304) (end 154.94 90.17) (width 0.254) (layer "B.Cu") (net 11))
 (segment (start 170.18 72.39) (end 168.6348 70.8448) (width 0.254) (layer "B.Cu") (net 2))
 (segment (start 160.2702 70.8448) (end 158.74 72.375) (width 0.254) (layer "B.Cu") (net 2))
 (segment (start 168.6348 70.8448) (end 160.2702 70.8448) (width 0.254) (layer "B.Cu") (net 2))
 (segment (start 167.64 80.01) (end 170.18 77.47) (width 0.254) (layer "B.Cu") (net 2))
 (segment (start 170.18 77.47) (end 170.18 72.39) (width 0.254) (layer "B.Cu") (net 2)))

